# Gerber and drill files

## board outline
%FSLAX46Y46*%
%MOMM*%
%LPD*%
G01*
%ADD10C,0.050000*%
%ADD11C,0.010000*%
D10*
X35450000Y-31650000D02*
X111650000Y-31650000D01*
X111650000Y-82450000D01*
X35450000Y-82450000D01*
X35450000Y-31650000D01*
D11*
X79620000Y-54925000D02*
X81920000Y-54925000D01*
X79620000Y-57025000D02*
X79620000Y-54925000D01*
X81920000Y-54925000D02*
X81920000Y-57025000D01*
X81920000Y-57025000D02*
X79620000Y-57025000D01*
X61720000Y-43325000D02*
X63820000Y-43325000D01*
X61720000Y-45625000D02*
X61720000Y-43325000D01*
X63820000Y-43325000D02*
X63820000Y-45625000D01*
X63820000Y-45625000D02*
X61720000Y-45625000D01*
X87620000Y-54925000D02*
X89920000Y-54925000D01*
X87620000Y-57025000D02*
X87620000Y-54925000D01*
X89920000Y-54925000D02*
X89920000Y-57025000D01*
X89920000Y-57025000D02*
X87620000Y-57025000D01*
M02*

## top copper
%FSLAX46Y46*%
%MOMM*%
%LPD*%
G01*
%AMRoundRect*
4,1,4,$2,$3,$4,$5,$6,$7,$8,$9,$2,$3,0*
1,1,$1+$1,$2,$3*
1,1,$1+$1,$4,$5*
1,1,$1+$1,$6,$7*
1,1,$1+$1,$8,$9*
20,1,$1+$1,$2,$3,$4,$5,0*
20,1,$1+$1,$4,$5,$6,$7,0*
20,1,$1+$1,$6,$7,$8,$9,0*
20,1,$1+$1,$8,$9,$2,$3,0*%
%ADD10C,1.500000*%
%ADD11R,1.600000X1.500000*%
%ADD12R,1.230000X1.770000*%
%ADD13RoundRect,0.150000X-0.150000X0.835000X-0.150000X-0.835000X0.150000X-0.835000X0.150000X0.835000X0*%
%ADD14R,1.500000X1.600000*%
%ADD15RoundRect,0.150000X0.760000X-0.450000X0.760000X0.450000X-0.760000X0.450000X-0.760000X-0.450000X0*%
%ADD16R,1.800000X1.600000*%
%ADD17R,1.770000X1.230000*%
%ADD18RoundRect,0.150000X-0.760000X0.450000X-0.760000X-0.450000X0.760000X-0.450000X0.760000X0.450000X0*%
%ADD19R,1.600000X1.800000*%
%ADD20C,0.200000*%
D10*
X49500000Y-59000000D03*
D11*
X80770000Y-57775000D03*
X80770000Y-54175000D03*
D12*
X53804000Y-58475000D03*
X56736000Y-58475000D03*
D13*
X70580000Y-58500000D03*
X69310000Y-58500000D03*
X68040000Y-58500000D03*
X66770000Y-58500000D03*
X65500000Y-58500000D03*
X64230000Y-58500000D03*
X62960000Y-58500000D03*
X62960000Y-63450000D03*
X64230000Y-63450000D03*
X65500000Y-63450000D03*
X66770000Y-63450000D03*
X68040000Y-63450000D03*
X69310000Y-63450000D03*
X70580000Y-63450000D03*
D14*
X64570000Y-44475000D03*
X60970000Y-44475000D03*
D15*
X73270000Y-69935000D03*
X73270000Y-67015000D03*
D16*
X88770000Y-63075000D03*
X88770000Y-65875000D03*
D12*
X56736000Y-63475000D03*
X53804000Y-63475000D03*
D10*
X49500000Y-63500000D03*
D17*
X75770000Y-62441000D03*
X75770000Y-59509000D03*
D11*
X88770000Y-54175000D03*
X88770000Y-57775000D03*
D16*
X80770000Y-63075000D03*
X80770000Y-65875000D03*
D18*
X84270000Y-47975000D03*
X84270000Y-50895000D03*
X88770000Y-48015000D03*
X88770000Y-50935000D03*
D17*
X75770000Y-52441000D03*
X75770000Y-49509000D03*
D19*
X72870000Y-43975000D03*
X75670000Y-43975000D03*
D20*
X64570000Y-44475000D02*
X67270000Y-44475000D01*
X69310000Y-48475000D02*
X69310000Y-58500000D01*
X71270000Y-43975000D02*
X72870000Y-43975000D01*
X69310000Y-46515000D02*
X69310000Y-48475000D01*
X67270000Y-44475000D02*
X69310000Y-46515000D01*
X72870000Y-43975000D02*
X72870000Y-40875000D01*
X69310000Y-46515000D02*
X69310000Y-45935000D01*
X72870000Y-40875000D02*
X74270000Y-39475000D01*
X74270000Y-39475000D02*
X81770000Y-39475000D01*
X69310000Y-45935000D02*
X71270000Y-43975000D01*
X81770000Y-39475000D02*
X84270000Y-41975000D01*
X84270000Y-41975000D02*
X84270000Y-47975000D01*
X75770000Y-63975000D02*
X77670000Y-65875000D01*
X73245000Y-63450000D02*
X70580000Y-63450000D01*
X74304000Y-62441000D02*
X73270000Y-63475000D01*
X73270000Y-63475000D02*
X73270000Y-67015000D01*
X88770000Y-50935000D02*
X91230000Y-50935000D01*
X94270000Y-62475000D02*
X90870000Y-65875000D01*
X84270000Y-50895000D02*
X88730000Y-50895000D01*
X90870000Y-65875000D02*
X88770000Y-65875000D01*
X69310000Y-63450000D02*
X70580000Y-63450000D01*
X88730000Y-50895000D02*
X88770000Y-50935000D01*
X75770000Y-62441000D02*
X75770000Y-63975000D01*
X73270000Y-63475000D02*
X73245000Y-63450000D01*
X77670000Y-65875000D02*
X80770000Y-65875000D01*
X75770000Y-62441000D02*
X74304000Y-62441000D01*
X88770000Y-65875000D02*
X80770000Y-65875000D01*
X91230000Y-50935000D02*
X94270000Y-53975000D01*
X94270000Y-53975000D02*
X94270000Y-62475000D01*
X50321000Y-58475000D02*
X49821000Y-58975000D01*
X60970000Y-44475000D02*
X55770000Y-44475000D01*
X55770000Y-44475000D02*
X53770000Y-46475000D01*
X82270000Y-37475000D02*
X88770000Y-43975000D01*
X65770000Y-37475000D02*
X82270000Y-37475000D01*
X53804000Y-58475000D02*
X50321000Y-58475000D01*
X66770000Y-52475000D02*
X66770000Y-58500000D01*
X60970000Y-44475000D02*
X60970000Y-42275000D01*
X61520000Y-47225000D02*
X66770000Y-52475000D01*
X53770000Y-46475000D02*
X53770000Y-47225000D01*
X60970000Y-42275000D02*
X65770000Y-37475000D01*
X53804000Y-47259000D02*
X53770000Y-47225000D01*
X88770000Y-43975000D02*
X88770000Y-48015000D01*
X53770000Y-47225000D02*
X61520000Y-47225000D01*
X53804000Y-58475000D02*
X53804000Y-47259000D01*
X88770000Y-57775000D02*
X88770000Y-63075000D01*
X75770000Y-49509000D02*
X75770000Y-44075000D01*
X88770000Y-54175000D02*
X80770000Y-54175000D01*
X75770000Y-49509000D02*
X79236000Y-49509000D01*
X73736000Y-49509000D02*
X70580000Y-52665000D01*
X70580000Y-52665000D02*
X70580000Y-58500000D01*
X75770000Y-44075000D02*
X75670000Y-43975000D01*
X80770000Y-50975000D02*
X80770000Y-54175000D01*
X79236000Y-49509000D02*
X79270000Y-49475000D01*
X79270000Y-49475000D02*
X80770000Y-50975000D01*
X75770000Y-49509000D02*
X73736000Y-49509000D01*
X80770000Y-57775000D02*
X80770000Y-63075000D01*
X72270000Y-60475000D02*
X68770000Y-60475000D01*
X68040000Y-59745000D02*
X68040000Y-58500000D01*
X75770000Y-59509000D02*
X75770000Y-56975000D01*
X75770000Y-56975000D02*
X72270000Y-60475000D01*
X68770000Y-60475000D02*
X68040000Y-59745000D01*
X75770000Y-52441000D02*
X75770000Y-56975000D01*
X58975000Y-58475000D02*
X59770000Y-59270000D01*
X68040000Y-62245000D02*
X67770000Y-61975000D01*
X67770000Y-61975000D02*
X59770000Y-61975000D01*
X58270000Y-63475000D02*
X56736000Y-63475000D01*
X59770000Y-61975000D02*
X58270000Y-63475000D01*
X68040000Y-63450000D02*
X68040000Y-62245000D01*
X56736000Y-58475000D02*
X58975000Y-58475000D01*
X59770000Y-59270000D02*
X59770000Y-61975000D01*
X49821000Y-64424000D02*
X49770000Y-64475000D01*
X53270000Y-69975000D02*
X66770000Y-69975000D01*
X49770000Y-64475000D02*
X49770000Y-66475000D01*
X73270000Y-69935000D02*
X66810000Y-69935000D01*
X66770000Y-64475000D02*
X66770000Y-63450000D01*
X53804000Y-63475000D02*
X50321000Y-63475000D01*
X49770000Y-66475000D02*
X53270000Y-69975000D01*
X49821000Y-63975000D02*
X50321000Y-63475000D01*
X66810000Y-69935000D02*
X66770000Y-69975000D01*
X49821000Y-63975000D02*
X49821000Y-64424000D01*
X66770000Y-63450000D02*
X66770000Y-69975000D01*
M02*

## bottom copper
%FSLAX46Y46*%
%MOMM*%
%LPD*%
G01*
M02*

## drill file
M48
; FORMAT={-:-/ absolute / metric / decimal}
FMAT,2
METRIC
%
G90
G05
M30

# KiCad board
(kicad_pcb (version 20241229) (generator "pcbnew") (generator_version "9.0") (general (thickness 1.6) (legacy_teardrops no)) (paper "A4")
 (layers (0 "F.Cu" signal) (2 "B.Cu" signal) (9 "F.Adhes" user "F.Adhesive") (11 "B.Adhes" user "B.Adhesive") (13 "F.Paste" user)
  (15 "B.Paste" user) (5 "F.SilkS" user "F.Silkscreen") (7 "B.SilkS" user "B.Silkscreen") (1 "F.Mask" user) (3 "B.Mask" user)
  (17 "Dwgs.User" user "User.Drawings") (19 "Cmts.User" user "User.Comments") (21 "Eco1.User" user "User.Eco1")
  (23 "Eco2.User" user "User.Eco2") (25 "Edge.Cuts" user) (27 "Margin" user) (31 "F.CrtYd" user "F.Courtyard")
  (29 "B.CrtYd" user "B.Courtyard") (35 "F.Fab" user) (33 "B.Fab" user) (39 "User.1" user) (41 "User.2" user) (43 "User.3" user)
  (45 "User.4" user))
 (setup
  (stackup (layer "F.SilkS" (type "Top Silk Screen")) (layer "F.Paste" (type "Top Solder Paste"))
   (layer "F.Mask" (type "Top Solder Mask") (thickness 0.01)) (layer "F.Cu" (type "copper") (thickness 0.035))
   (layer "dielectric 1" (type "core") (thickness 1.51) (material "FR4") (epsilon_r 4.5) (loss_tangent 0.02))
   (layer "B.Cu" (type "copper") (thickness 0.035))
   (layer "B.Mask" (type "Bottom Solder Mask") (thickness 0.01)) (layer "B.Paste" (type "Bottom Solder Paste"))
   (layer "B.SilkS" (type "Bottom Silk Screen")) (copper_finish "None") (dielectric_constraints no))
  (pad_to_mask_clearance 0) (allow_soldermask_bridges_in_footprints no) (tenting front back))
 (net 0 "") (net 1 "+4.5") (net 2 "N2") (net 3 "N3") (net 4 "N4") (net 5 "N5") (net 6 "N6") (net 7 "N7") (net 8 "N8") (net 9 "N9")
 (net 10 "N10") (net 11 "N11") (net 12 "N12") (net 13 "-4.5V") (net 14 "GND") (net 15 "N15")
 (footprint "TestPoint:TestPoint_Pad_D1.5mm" (layer "F.Cu") (at 49.5 59)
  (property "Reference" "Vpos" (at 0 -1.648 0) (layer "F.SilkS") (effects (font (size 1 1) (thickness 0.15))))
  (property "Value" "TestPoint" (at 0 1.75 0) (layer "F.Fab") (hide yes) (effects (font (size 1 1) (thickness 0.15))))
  (pad "1" smd circle (at 0 0) (size 1.5 1.5) (layers "F.Cu" "F.Mask") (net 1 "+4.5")))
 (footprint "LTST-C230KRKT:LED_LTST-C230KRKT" (layer "F.Cu") (at 80.77 55.975 -90)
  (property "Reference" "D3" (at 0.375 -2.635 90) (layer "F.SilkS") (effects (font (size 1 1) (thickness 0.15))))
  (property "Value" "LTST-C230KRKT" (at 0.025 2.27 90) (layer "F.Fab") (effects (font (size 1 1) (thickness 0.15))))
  (fp_line (start -1.05 1.15) (end -1.05 -1.15) (stroke (width 0.01) (type solid)) (layer "Edge.Cuts"))
  (fp_line (start 1.05 1.15) (end -1.05 1.15) (stroke (width 0.01) (type solid)) (layer "Edge.Cuts"))
  (fp_line (start -1.05 -1.15) (end 1.05 -1.15) (stroke (width 0.01) (type solid)) (layer "Edge.Cuts"))
  (fp_line (start 1.05 -1.15) (end 1.05 1.15) (stroke (width 0.01) (type solid)) (layer "Edge.Cuts"))
  (pad "A" smd rect (at 1.8 0 270) (size 1.5 1.6) (layers "F.Cu" "F.Mask" "F.Paste") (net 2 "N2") (solder_mask_margin 0.102))
  (pad "C" smd rect (at -1.8 0 270) (size 1.5 1.6) (layers "F.Cu" "F.Mask" "F.Paste") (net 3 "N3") (solder_mask_margin 0.102)))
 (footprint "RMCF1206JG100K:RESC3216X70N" (layer "F.Cu") (at 55.27 58.475)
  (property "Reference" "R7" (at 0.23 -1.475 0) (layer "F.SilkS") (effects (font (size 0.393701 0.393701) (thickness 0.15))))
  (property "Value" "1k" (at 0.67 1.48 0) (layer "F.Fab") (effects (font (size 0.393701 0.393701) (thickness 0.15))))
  (pad "1" smd rect (at -1.466 0) (size 1.23 1.77) (layers "F.Cu" "F.Mask" "F.Paste") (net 1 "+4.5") (solder_mask_margin 0.102))
  (pad "2" smd rect (at 1.466 0) (size 1.23 1.77) (layers "F.Cu" "F.Mask" "F.Paste") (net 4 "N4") (solder_mask_margin 0.102)))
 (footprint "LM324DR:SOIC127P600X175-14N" (layer "F.Cu") (at 66.77 60.975 -90)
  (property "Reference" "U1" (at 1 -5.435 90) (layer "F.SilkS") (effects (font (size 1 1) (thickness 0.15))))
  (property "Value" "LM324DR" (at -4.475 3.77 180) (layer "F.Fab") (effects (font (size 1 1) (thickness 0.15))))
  (pad "1" smd roundrect (at -2.475 -3.81 270) (size 1.97 0.6) (layers "F.Cu" "F.Mask" "F.Paste") (roundrect_rratio 0.25) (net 3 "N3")
   (solder_mask_margin 0.102))
  (pad "2" smd roundrect (at -2.475 -2.54 270) (size 1.97 0.6) (layers "F.Cu" "F.Mask" "F.Paste") (roundrect_rratio 0.25) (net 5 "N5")
   (solder_mask_margin 0.102))
  (pad "3" smd roundrect (at -2.475 -1.27 270) (size 1.97 0.6) (layers "F.Cu" "F.Mask" "F.Paste") (roundrect_rratio 0.25) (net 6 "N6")
   (solder_mask_margin 0.102))
  (pad "4" smd roundrect (at -2.475 0 270) (size 1.97 0.6) (layers "F.Cu" "F.Mask" "F.Paste") (roundrect_rratio 0.25) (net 1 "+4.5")
   (solder_mask_margin 0.102))
  (pad "5" smd roundrect (at -2.475 1.27 270) (size 1.97 0.6) (layers "F.Cu" "F.Mask" "F.Paste") (roundrect_rratio 0.25) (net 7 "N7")
   (solder_mask_margin 0.102))
  (pad "6" smd roundrect (at -2.475 2.54 270) (size 1.97 0.6) (layers "F.Cu" "F.Mask" "F.Paste") (roundrect_rratio 0.25) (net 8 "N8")
   (solder_mask_margin 0.102))
  (pad "7" smd roundrect (at -2.475 3.81 270) (size 1.97 0.6) (layers "F.Cu" "F.Mask" "F.Paste") (roundrect_rratio 0.25) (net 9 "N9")
   (solder_mask_margin 0.102))
  (pad "8" smd roundrect (at 2.475 3.81 270) (size 1.97 0.6) (layers "F.Cu" "F.Mask" "F.Paste") (roundrect_rratio 0.25) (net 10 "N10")
   (solder_mask_margin 0.102))
  (pad "9" smd roundrect (at 2.475 2.54 270) (size 1.97 0.6) (layers "F.Cu" "F.Mask" "F.Paste") (roundrect_rratio 0.25) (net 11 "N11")
   (solder_mask_margin 0.102))
  (pad "10" smd roundrect (at 2.475 1.27 270) (size 1.97 0.6) (layers "F.Cu" "F.Mask" "F.Paste") (roundrect_rratio 0.25) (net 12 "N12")
   (solder_mask_margin 0.102))
  (pad "11" smd roundrect (at 2.475 0 270) (size 1.97 0.6) (layers "F.Cu" "F.Mask" "F.Paste") (roundrect_rratio 0.25) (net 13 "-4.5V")
   (solder_mask_margin 0.102))
  (pad "12" smd roundrect (at 2.475 -1.27 270) (size 1.97 0.6) (layers "F.Cu" "F.Mask" "F.Paste") (roundrect_rratio 0.25) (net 4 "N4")
   (solder_mask_margin 0.102))
  (pad "13" smd roundrect (at 2.475 -2.54 270) (size 1.97 0.6) (layers "F.Cu" "F.Mask" "F.Paste") (roundrect_rratio 0.25) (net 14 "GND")
   (solder_mask_margin 0.102))
  (pad "14" smd roundrect (at 2.475 -3.81 270) (size 1.97 0.6) (layers "F.Cu" "F.Mask" "F.Paste") (roundrect_rratio 0.25) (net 14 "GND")
   (solder_mask_margin 0.102)))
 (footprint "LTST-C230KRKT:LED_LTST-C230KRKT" (layer "F.Cu") (at 62.77 44.475)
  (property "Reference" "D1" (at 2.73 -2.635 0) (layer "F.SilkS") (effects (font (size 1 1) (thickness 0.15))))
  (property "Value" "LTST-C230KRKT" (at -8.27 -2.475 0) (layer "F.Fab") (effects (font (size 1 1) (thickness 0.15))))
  (fp_line (start -1.05 -1.15) (end 1.05 -1.15) (stroke (width 0.01) (type solid)) (layer "Edge.Cuts"))
  (fp_line (start -1.05 1.15) (end -1.05 -1.15) (stroke (width 0.01) (type solid)) (layer "Edge.Cuts"))
  (fp_line (start 1.05 -1.15) (end 1.05 1.15) (stroke (width 0.01) (type solid)) (layer "Edge.Cuts"))
  (fp_line (start 1.05 1.15) (end -1.05 1.15) (stroke (width 0.01) (type solid)) (layer "Edge.Cuts"))
  (pad "A" smd rect (at 1.8 0) (size 1.5 1.6) (layers "F.Cu" "F.Mask" "F.Paste") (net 5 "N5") (solder_mask_margin 0.102))
  (pad "C" smd rect (at -1.8 0) (size 1.5 1.6) (layers "F.Cu" "F.Mask" "F.Paste") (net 1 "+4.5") (solder_mask_margin 0.102)))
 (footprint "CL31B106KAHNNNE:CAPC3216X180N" (layer "F.Cu") (at 73.27 68.475 90)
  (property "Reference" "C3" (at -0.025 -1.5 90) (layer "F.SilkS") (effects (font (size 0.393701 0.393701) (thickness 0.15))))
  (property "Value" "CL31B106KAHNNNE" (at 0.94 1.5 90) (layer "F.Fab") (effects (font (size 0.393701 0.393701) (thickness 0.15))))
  (pad "1" smd roundrect (at -1.46 0 90) (size 1.2 1.82) (layers "F.Cu" "F.Mask" "F.Paste") (roundrect_rratio 0.125) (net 13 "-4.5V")
   (solder_mask_margin 0.102))
  (pad "2" smd roundrect (at 1.46 0 90) (size 1.2 1.82) (layers "F.Cu" "F.Mask" "F.Paste") (roundrect_rratio 0.125) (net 14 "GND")
   (solder_mask_margin 0.102)))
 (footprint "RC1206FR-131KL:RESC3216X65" (layer "F.Cu") (at 88.77 64.475 -90)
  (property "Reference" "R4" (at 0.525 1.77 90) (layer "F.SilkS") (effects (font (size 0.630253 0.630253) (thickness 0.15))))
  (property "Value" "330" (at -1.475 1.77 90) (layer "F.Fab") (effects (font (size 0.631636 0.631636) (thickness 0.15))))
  (pad "1" smd rect (at -1.4 0 270) (size 1.6 1.8) (layers "F.Cu" "F.Mask" "F.Paste") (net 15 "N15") (solder_mask_margin 0.102))
  (pad "2" smd rect (at 1.4 0 270) (size 1.6 1.8) (layers "F.Cu" "F.Mask" "F.Paste") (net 14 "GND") (solder_mask_margin 0.102)))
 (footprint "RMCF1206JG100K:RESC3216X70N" (layer "F.Cu") (at 55.27 63.475 180)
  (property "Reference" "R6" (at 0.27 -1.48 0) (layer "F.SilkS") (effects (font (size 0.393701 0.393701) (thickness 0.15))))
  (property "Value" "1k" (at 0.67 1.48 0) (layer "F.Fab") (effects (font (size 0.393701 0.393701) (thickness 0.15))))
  (pad "1" smd rect (at -1.466 0 180) (size 1.23 1.77) (layers "F.Cu" "F.Mask" "F.Paste") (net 4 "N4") (solder_mask_margin 0.102))
  (pad "2" smd rect (at 1.466 0 180) (size 1.23 1.77) (layers "F.Cu" "F.Mask" "F.Paste") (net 13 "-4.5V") (solder_mask_margin 0.102)))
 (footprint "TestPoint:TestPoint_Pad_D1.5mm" (layer "F.Cu") (at 49.5 63.5)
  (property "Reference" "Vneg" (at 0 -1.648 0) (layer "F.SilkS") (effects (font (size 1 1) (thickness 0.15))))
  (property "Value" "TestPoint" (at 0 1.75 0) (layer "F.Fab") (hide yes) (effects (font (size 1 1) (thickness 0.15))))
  (pad "1" smd circle (at 0 0) (size 1.5 1.5) (layers "F.Cu" "F.Mask") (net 13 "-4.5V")))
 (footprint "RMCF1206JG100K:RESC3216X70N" (layer "F.Cu") (at 75.77 60.975 90)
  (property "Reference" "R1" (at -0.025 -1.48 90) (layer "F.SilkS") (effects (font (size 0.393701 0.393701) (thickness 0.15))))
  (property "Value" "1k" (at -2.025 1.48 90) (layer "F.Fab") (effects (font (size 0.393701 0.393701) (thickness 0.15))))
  (pad "1" smd rect (at -1.466 0 90) (size 1.23 1.77) (layers "F.Cu" "F.Mask" "F.Paste") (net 14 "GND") (solder_mask_margin 0.102))
  (pad "2" smd rect (at 1.466 0 90) (size 1.23 1.77) (layers "F.Cu" "F.Mask" "F.Paste") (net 6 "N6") (solder_mask_margin 0.102)))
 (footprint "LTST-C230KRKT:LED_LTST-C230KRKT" (layer "F.Cu") (at 88.77 55.975 90)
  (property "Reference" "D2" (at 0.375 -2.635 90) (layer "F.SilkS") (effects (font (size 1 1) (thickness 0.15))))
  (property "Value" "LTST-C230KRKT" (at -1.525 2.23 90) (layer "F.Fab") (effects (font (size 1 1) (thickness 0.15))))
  (fp_line (start 1.05 -1.15) (end 1.05 1.15) (stroke (width 0.01) (type solid)) (layer "Edge.Cuts"))
  (fp_line (start -1.05 -1.15) (end 1.05 -1.15) (stroke (width 0.01) (type solid)) (layer "Edge.Cuts"))
  (fp_line (start 1.05 1.15) (end -1.05 1.15) (stroke (width 0.01) (type solid)) (layer "Edge.Cuts"))
  (fp_line (start -1.05 1.15) (end -1.05 -1.15) (stroke (width 0.01) (type solid)) (layer "Edge.Cuts"))
  (pad "A" smd rect (at 1.8 0 90) (size 1.5 1.6) (layers "F.Cu" "F.Mask" "F.Paste") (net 3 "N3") (solder_mask_margin 0.102))
  (pad "C" smd rect (at -1.8 0 90) (size 1.5 1.6) (layers "F.Cu" "F.Mask" "F.Paste") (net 15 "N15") (solder_mask_margin 0.102)))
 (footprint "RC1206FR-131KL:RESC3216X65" (layer "F.Cu") (at 80.77 64.475 -90)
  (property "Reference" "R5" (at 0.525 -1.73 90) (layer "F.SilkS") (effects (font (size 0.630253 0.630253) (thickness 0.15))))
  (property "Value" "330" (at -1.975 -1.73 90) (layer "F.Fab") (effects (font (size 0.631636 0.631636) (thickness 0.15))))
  (pad "1" smd rect (at -1.4 0 270) (size 1.6 1.8) (layers "F.Cu" "F.Mask" "F.Paste") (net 2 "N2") (solder_mask_margin 0.102))
  (pad "2" smd rect (at 1.4 0 270) (size 1.6 1.8) (layers "F.Cu" "F.Mask" "F.Paste") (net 14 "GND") (solder_mask_margin 0.102)))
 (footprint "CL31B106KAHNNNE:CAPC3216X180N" (layer "F.Cu") (at 84.27 49.435 -90)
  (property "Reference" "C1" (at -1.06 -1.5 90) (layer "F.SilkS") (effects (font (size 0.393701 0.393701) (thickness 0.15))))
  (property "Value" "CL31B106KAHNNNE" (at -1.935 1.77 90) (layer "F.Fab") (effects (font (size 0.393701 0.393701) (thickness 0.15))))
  (pad "1" smd roundrect (at -1.46 0 270) (size 1.2 1.82) (layers "F.Cu" "F.Mask" "F.Paste") (roundrect_rratio 0.125) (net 5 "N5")
   (solder_mask_margin 0.102))
  (pad "2" smd roundrect (at 1.46 0 270) (size 1.2 1.82) (layers "F.Cu" "F.Mask" "F.Paste") (roundrect_rratio 0.125) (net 14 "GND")
   (solder_mask_margin 0.102)))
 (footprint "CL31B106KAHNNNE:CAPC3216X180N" (layer "F.Cu") (at 88.77 49.475 -90)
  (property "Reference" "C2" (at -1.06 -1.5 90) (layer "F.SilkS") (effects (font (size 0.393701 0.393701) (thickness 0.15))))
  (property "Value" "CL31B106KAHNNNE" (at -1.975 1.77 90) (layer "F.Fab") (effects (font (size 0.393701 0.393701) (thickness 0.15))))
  (pad "1" smd roundrect (at -1.46 0 270) (size 1.2 1.82) (layers "F.Cu" "F.Mask" "F.Paste") (roundrect_rratio 0.125) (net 1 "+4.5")
   (solder_mask_margin 0.102))
  (pad "2" smd roundrect (at 1.46 0 270) (size 1.2 1.82) (layers "F.Cu" "F.Mask" "F.Paste") (roundrect_rratio 0.125) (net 14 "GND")
   (solder_mask_margin 0.102)))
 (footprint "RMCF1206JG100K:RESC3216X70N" (layer "F.Cu") (at 75.77 50.975 90)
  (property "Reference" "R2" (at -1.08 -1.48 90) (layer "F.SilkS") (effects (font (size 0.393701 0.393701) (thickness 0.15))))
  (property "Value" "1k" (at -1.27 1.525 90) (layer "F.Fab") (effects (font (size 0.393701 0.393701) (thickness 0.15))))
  (pad "1" smd rect (at -1.466 0 90) (size 1.23 1.77) (layers "F.Cu" "F.Mask" "F.Paste") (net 6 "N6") (solder_mask_margin 0.102))
  (pad "2" smd rect (at 1.466 0 90) (size 1.23 1.77) (layers "F.Cu" "F.Mask" "F.Paste") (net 3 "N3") (solder_mask_margin 0.102)))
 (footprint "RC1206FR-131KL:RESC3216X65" (layer "F.Cu") (at 74.27 43.975)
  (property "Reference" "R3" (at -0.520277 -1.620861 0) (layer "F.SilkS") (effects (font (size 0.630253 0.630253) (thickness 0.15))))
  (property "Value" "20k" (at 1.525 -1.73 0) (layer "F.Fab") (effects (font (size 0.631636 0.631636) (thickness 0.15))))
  (pad "1" smd rect (at -1.4 0) (size 1.6 1.8) (layers "F.Cu" "F.Mask" "F.Paste") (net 5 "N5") (solder_mask_margin 0.102))
  (pad "2" smd rect (at 1.4 0) (size 1.6 1.8) (layers "F.Cu" "F.Mask" "F.Paste") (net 3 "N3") (solder_mask_margin 0.102)))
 (gr_rect (start 35.45 31.65) (end 111.65 82.45) (stroke (width 0.05) (type solid)) (fill no) (layer "Edge.Cuts"))
 (segment (start 64.57 44.475) (end 67.27 44.475) (width 0.2) (layer "F.Cu") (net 5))
 (segment (start 69.31 48.475) (end 69.31 58.5) (width 0.2) (layer "F.Cu") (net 5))
 (segment (start 71.27 43.975) (end 72.87 43.975) (width 0.2) (layer "F.Cu") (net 5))
 (segment (start 69.31 46.515) (end 69.31 48.475) (width 0.2) (layer "F.Cu") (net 5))
 (segment (start 67.27 44.475) (end 69.31 46.515) (width 0.2) (layer "F.Cu") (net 5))
 (segment (start 72.87 43.975) (end 72.87 40.875) (width 0.2) (layer "F.Cu") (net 5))
 (segment (start 69.31 46.515) (end 69.31 45.935) (width 0.2) (layer "F.Cu") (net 5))
 (segment (start 72.87 40.875) (end 74.27 39.475) (width 0.2) (layer "F.Cu") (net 5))
 (segment (start 74.27 39.475) (end 81.77 39.475) (width 0.2) (layer "F.Cu") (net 5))
 (segment (start 69.31 45.935) (end 71.27 43.975) (width 0.2) (layer "F.Cu") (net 5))
 (segment (start 81.77 39.475) (end 84.27 41.975) (width 0.2) (layer "F.Cu") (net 5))
 (segment (start 84.27 41.975) (end 84.27 47.975) (width 0.2) (layer "F.Cu") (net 5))
 (segment (start 75.77 63.975) (end 77.67 65.875) (width 0.2) (layer "F.Cu") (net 14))
 (segment (start 73.245 63.45) (end 70.58 63.45) (width 0.2) (layer "F.Cu") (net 14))
 (segment (start 74.304 62.441) (end 73.27 63.475) (width 0.2) (layer "F.Cu") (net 14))
 (segment (start 73.27 63.475) (end 73.27 67.015) (width 0.2) (layer "F.Cu") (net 14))
 (segment (start 88.77 50.935) (end 91.23 50.935) (width 0.2) (layer "F.Cu") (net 14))
 (segment (start 94.27 62.475) (end 90.87 65.875) (width 0.2) (layer "F.Cu") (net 14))
 (segment (start 84.27 50.895) (end 88.73 50.895) (width 0.2) (layer "F.Cu") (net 14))
 (segment (start 90.87 65.875) (end 88.77 65.875) (width 0.2) (layer "F.Cu") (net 14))
 (segment (start 69.31 63.45) (end 70.58 63.45) (width 0.2) (layer "F.Cu") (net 14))
 (segment (start 88.73 50.895) (end 88.77 50.935) (width 0.2) (layer "F.Cu") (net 14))
 (segment (start 75.77 62.441) (end 75.77 63.975) (width 0.2) (layer "F.Cu") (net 14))
 (segment (start 73.27 63.475) (end 73.245 63.45) (width 0.2) (layer "F.Cu") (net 14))
 (segment (start 77.67 65.875) (end 80.77 65.875) (width 0.2) (layer "F.Cu") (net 14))
 (segment (start 75.77 62.441) (end 74.304 62.441) (width 0.2) (layer "F.Cu") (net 14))
 (segment (start 88.77 65.875) (end 80.77 65.875) (width 0.2) (layer "F.Cu") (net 14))
 (segment (start 91.23 50.935) (end 94.27 53.975) (width 0.2) (layer "F.Cu") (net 14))
 (segment (start 94.27 53.975) (end 94.27 62.475) (width 0.2) (layer "F.Cu") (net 14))
 (segment (start 50.321 58.475) (end 49.821 58.975) (width 0.2) (layer "F.Cu") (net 1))
 (segment (start 60.97 44.475) (end 55.77 44.475) (width 0.2) (layer "F.Cu") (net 1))
 (segment (start 55.77 44.475) (end 53.77 46.475) (width 0.2) (layer "F.Cu") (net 1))
 (segment (start 82.27 37.475) (end 88.77 43.975) (width 0.2) (layer "F.Cu") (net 1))
 (segment (start 65.77 37.475) (end 82.27 37.475) (width 0.2) (layer "F.Cu") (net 1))
 (segment (start 53.804 58.475) (end 50.321 58.475) (width 0.2) (layer "F.Cu") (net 1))
 (segment (start 66.77 52.475) (end 66.77 58.5) (width 0.2) (layer "F.Cu") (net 1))
 (segment (start 60.97 44.475) (end 60.97 42.275) (width 0.2) (layer "F.Cu") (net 1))
 (segment (start 61.52 47.225) (end 66.77 52.475) (width 0.2) (layer "F.Cu") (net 1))
 (segment (start 53.77 46.475) (end 53.77 47.225) (width 0.2) (layer "F.Cu") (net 1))
 (segment (start 60.97 42.275) (end 65.77 37.475) (width 0.2) (layer "F.Cu") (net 1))
 (segment (start 53.804 47.259) (end 53.77 47.225) (width 0.2) (layer "F.Cu") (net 1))
 (segment (start 88.77 43.975) (end 88.77 48.015) (width 0.2) (layer "F.Cu") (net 1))
 (segment (start 53.77 47.225) (end 61.52 47.225) (width 0.2) (layer "F.Cu") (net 1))
 (segment (start 53.804 58.475) (end 53.804 47.259) (width 0.2) (layer "F.Cu") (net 1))
 (segment (start 88.77 57.775) (end 88.77 63.075) (width 0.2) (layer "F.Cu") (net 15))
 (segment (start 75.77 49.509) (end 75.77 44.075) (width 0.2) (layer "F.Cu") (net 3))
 (segment (start 88.77 54.175) (end 80.77 54.175) (width 0.2) (layer "F.Cu") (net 3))
 (segment (start 75.77 49.509) (end 79.236 49.509) (width 0.2) (layer "F.Cu") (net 3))
 (segment (start 73.736 49.509) (end 70.58 52.665) (width 0.2) (layer "F.Cu") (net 3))
 (segment (start 70.58 52.665) (end 70.58 58.5) (width 0.2) (layer "F.Cu") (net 3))
 (segment (start 75.77 44.075) (end 75.67 43.975) (width 0.2) (layer "F.Cu") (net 3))
 (segment (start 80.77 50.975) (end 80.77 54.175) (width 0.2) (layer "F.Cu") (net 3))
 (segment (start 79.236 49.509) (end 79.27 49.475) (width 0.2) (layer "F.Cu") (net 3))
 (segment (start 79.27 49.475) (end 80.77 50.975) (width 0.2) (layer "F.Cu") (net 3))
 (segment (start 75.77 49.509) (end 73.736 49.509) (width 0.2) (layer "F.Cu") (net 3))
 (segment (start 80.77 57.775) (end 80.77 63.075) (width 0.2) (layer "F.Cu") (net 2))
 (segment (start 72.27 60.475) (end 68.77 60.475) (width 0.2) (layer "F.Cu") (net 6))
 (segment (start 68.04 59.745) (end 68.04 58.5) (width 0.2) (layer "F.Cu") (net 6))
 (segment (start 75.77 59.509) (end 75.77 56.975) (width 0.2) (layer "F.Cu") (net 6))
 (segment (start 75.77 56.975) (end 72.27 60.475) (width 0.2) (layer "F.Cu") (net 6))
 (segment (start 68.77 60.475) (end 68.04 59.745) (width 0.2) (layer "F.Cu") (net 6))
 (segment (start 75.77 52.441) (end 75.77 56.975) (width 0.2) (layer "F.Cu") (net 6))
 (segment (start 58.975 58.475) (end 59.77 59.27) (width 0.2) (layer "F.Cu") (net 4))
 (segment (start 68.04 62.245) (end 67.77 61.975) (width 0.2) (layer "F.Cu") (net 4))
 (segment (start 67.77 61.975) (end 59.77 61.975) (width 0.2) (layer "F.Cu") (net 4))
 (segment (start 58.27 63.475) (end 56.736 63.475) (width 0.2) (layer "F.Cu") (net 4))
 (segment (start 59.77 61.975) (end 58.27 63.475) (width 0.2) (layer "F.Cu") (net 4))
 (segment (start 68.04 63.45) (end 68.04 62.245) (width 0.2) (layer "F.Cu") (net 4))
 (segment (start 56.736 58.475) (end 58.975 58.475) (width 0.2) (layer "F.Cu") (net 4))
 (segment (start 59.77 59.27) (end 59.77 61.975) (width 0.2) (layer "F.Cu") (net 4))
 (segment (start 49.821 64.424) (end 49.77 64.475) (width 0.2) (layer "F.Cu") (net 13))
 (segment (start 53.27 69.975) (end 66.77 69.975) (width 0.2) (layer "F.Cu") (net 13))
 (segment (start 49.77 64.475) (end 49.77 66.475) (width 0.2) (layer "F.Cu") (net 13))
 (segment (start 73.27 69.935) (end 66.81 69.935) (width 0.2) (layer "F.Cu") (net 13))
 (segment (start 66.77 64.475) (end 66.77 63.45) (width 0.2) (layer "F.Cu") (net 13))
 (segment (start 53.804 63.475) (end 50.321 63.475) (width 0.2) (layer "F.Cu") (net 13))
 (segment (start 49.77 66.475) (end 53.27 69.975) (width 0.2) (layer "F.Cu") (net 13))
 (segment (start 49.821 63.975) (end 50.321 63.475) (width 0.2) (layer "F.Cu") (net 13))
 (segment (start 66.81 69.935) (end 66.77 69.975) (width 0.2) (layer "F.Cu") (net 13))
 (segment (start 49.821 63.975) (end 49.821 64.424) (width 0.2) (layer "F.Cu") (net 13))
 (segment (start 66.77 63.45) (end 66.77 69.975) (width 0.2) (layer "F.Cu") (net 13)))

